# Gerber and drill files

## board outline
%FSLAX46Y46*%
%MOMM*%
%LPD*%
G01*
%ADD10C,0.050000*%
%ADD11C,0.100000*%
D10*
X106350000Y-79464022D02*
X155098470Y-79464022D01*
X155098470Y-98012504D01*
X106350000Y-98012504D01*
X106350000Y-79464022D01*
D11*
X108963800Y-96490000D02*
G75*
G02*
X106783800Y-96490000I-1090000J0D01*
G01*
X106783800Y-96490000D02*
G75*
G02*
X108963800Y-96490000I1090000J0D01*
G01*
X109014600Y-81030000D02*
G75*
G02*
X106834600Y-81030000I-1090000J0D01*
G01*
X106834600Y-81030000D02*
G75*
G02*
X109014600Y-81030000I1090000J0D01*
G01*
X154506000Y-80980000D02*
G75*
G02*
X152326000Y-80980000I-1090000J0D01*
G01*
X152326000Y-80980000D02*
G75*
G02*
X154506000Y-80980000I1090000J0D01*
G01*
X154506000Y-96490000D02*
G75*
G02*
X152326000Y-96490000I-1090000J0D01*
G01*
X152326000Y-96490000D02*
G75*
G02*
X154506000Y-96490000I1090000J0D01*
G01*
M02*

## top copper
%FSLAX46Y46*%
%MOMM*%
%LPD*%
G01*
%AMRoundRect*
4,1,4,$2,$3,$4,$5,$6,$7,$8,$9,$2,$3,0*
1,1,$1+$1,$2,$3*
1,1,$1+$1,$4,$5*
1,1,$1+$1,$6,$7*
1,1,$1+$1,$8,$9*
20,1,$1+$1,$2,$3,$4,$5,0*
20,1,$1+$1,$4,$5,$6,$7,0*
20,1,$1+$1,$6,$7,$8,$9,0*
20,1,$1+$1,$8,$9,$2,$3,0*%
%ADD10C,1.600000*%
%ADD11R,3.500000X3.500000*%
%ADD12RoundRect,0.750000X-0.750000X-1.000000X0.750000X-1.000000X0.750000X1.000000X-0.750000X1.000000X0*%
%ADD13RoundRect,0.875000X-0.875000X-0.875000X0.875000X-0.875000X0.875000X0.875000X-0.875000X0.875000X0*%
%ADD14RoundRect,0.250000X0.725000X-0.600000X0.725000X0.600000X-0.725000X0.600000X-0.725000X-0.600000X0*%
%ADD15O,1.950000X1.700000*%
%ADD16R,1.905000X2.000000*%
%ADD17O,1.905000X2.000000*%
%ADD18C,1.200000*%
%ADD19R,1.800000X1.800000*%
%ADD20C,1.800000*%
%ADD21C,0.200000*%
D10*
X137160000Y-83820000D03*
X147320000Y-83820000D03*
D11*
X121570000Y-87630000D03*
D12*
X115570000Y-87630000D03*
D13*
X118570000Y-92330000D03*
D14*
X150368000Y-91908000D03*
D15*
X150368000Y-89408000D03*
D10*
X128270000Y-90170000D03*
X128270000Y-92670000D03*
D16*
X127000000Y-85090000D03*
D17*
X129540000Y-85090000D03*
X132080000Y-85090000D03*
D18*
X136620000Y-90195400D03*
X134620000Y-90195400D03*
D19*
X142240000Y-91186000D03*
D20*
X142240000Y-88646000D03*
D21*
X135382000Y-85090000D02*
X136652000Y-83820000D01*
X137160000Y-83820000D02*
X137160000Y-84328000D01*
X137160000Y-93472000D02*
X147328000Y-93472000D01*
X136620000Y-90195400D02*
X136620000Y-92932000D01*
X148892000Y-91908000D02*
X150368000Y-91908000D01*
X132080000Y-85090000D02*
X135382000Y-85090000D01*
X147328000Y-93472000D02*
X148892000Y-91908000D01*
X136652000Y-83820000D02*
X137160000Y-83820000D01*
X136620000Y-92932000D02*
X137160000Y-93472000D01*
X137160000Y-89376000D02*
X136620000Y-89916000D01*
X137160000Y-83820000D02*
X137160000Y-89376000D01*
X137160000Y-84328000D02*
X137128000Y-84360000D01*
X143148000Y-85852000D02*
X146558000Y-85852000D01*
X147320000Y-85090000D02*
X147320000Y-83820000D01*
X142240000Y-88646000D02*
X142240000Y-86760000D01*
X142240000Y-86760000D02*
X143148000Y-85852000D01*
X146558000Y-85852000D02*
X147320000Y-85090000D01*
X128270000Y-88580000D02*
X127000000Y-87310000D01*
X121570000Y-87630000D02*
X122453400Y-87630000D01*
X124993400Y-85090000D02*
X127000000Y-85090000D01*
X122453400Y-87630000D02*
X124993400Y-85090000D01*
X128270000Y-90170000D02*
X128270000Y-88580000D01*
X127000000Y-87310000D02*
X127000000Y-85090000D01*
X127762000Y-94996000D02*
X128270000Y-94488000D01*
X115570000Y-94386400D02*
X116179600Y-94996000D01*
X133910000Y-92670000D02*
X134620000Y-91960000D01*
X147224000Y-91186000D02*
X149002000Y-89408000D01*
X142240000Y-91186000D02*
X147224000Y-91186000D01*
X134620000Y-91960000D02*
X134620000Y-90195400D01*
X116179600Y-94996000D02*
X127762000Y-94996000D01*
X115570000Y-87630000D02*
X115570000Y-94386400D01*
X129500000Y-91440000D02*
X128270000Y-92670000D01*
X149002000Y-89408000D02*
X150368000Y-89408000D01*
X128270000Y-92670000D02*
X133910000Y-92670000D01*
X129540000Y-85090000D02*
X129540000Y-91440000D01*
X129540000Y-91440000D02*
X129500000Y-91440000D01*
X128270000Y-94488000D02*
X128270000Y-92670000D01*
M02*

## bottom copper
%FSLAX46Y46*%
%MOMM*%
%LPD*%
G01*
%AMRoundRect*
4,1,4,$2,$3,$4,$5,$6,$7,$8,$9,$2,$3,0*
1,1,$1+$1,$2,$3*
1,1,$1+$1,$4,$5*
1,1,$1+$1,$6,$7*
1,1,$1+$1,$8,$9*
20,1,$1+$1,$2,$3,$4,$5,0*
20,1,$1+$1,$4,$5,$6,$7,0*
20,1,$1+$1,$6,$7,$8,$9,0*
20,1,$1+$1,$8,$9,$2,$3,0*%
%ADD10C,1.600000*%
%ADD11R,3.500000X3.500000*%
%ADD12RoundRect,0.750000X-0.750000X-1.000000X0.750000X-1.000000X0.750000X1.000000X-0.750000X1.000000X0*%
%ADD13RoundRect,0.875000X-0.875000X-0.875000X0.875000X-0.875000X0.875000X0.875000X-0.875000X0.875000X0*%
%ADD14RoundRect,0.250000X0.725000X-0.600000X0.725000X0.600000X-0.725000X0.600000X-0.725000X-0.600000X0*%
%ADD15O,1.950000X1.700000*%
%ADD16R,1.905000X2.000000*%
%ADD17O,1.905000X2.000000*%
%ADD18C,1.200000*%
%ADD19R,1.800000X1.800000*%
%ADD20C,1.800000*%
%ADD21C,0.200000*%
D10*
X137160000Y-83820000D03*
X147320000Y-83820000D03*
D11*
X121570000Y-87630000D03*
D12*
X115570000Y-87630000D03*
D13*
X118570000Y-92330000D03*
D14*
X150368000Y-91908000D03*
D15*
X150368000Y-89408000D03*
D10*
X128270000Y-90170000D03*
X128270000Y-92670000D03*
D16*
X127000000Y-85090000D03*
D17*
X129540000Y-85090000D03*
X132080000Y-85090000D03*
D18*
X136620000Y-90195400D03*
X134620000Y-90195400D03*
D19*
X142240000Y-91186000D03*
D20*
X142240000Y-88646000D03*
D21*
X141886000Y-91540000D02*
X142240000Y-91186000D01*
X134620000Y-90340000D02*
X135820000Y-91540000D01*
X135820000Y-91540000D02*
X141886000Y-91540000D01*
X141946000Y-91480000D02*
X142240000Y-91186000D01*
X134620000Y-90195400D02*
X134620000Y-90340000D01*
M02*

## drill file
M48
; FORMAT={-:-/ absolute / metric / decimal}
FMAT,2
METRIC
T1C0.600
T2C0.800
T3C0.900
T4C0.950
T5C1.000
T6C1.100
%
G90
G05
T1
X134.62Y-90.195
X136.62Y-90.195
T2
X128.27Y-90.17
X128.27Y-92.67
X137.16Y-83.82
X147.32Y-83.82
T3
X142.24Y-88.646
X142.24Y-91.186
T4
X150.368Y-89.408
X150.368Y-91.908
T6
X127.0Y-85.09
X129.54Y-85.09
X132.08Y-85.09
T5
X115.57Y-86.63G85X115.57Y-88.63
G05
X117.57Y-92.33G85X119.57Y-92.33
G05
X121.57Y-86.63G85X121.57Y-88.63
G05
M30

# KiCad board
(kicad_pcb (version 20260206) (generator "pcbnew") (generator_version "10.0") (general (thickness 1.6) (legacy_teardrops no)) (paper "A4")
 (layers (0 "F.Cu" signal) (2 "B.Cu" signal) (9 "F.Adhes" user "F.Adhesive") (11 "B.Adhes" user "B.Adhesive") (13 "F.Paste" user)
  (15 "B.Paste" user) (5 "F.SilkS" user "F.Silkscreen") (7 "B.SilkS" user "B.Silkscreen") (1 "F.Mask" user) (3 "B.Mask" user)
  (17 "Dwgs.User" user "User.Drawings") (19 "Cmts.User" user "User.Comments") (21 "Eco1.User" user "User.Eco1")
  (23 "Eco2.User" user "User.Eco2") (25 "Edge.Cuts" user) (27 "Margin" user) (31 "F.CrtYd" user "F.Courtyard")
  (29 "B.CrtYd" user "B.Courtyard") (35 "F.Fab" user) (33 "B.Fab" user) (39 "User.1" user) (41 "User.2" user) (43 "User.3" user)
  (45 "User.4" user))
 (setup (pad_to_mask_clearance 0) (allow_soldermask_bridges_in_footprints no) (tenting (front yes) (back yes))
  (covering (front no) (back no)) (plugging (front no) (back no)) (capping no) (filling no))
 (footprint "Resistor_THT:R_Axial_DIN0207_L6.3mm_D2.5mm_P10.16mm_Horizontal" (layer "F.Cu") (at 137.16 83.82)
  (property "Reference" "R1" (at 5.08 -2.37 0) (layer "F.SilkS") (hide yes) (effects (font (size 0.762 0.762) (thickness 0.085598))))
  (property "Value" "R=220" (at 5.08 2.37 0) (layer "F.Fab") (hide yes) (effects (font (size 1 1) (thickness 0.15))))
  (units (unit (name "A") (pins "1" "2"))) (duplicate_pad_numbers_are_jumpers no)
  (pad "1" thru_hole circle (at 0 0) (size 1.6 1.6) (drill 0.8) (layers "*.Cu" "*.Mask") (remove_unused_layers no) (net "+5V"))
  (pad "2" thru_hole circle (at 10.16 0) (size 1.6 1.6) (drill 0.8) (layers "*.Cu" "*.Mask") (remove_unused_layers no) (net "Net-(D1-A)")))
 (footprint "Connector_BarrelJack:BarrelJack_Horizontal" (layer "F.Cu") (at 121.57 87.63)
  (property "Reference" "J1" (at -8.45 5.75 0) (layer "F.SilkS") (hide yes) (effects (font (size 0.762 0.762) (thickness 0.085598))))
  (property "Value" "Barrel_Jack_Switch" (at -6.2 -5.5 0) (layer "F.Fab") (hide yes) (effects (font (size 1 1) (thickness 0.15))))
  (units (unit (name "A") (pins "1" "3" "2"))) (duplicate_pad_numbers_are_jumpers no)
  (pad "1" thru_hole rect (at 0 0) (size 3.5 3.5) (drill oval 1 3) (layers "*.Cu" "*.Mask") (remove_unused_layers no) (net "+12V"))
  (pad "2" thru_hole roundrect (at -6 0) (size 3 3.5) (drill oval 1 3) (layers "*.Cu" "*.Mask") (remove_unused_layers no)
   (roundrect_rratio 0.25) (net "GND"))
  (pad "3" thru_hole roundrect (at -3 4.7) (size 3.5 3.5) (drill oval 3 1) (layers "*.Cu" "*.Mask") (remove_unused_layers no)
   (roundrect_rratio 0.25) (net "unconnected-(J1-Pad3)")))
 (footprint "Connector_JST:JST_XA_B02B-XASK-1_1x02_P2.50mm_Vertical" (layer "F.Cu") (at 150.368 91.908 90)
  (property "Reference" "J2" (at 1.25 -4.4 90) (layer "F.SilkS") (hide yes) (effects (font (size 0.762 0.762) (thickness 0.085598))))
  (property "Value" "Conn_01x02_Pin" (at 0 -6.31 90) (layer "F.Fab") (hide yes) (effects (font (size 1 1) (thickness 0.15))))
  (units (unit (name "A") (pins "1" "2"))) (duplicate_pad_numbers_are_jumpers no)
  (pad "1" thru_hole roundrect (at 0 0 90) (size 1.7 1.95) (drill 0.95) (layers "*.Cu" "*.Mask") (remove_unused_layers no)
   (roundrect_rratio 0.147059) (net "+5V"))
  (pad "2" thru_hole oval (at 2.5 0 90) (size 1.7 1.95) (drill 0.95) (layers "*.Cu" "*.Mask") (remove_unused_layers no) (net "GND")))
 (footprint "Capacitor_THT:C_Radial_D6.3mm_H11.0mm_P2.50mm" (layer "F.Cu") (at 128.27 90.17 -90)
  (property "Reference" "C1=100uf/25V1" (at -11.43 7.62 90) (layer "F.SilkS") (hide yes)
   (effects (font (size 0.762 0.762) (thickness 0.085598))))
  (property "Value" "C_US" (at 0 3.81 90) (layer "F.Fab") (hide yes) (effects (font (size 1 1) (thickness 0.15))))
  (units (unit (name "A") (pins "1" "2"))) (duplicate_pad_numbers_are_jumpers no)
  (pad "1" thru_hole circle (at 0 0 270) (size 1.6 1.6) (drill 0.8) (layers "*.Cu" "*.Mask") (remove_unused_layers no) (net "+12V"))
  (pad "2" thru_hole circle (at 2.5 0 270) (size 1.6 1.6) (drill 0.8) (layers "*.Cu" "*.Mask") (remove_unused_layers no) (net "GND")))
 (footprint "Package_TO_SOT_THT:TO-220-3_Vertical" (layer "F.Cu") (at 127 85.09)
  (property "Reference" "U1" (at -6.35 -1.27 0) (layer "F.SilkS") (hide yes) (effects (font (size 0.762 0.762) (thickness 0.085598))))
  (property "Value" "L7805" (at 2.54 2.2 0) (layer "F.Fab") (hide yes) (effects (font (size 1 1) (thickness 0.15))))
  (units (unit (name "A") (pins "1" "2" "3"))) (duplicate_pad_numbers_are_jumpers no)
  (pad "1" thru_hole rect (at 0 0) (size 1.905 2) (drill 1.1) (layers "*.Cu" "*.Mask") (remove_unused_layers no) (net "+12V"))
  (pad "2" thru_hole oval (at 2.54 0) (size 1.905 2) (drill 1.1) (layers "*.Cu" "*.Mask") (remove_unused_layers no) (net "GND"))
  (pad "3" thru_hole oval (at 5.08 0) (size 1.905 2) (drill 1.1) (layers "*.Cu" "*.Mask") (remove_unused_layers no) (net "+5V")))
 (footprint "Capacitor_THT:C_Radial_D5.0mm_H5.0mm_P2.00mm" (layer "F.Cu") (at 136.62 90.1954 180)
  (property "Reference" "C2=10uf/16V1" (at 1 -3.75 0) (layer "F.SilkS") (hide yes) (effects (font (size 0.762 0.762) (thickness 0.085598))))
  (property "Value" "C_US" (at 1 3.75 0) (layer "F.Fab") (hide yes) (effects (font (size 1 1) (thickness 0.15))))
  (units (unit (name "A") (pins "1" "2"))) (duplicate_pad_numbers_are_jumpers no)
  (pad "1" thru_hole circle (at 0 0 180) (size 1.2 1.2) (drill 0.6) (layers "*.Cu" "*.Mask") (remove_unused_layers no) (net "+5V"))
  (pad "2" thru_hole circle (at 2 0 180) (size 1.2 1.2) (drill 0.6) (layers "*.Cu" "*.Mask") (remove_unused_layers no) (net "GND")))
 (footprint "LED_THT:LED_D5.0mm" (layer "F.Cu") (at 142.24 91.186 90)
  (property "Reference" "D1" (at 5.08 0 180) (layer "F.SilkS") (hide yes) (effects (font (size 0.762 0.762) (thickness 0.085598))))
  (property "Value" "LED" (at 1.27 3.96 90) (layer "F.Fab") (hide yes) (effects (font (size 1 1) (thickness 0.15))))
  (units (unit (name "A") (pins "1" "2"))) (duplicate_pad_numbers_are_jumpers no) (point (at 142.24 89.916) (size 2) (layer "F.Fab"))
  (pad "1" thru_hole rect (at 0 0 90) (size 1.8 1.8) (drill 0.9) (layers "*.Cu" "*.Mask") (remove_unused_layers no) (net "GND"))
  (pad "2" thru_hole circle (at 2.54 0 90) (size 1.8 1.8) (drill 0.9) (layers "*.Cu" "*.Mask") (remove_unused_layers no) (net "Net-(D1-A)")))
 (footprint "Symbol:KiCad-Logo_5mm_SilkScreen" (layer "B.Cu") (at 110.71 88.35 90)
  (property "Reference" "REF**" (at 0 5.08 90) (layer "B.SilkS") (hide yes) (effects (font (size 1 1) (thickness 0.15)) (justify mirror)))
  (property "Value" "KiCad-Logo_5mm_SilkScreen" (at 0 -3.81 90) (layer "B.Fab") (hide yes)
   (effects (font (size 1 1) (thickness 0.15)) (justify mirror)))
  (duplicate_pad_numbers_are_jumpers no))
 (gr_rect (start 106.35 79.464022) (end 155.09847 98.012504) (stroke (width 0.05) (type default)) (fill no) (layer "Edge.Cuts"))
 (gr_circle (center 107.8738 96.49) (end 108.9638 96.49) (stroke (width 0.1) (type solid)) (fill no) (layer "Edge.Cuts"))
 (gr_circle (center 107.9246 81.03) (end 109.0146 81.03) (stroke (width 0.1) (type solid)) (fill no) (layer "Edge.Cuts"))
 (gr_circle (center 153.416 80.98) (end 154.506 80.98) (stroke (width 0.1) (type solid)) (fill no) (layer "Edge.Cuts"))
 (gr_circle (center 153.416 96.49) (end 153.416 97.58) (stroke (width 0.1) (type solid)) (fill no) (layer "Edge.Cuts"))
 (segment (start 135.382 85.09) (end 136.652 83.82) (width 0.2) (layer "F.Cu") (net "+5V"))
 (segment (start 137.16 83.82) (end 137.16 84.328) (width 0.2) (layer "F.Cu") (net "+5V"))
 (segment (start 137.16 93.472) (end 147.328 93.472) (width 0.2) (layer "F.Cu") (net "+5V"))
 (segment (start 136.62 90.1954) (end 136.62 92.932) (width 0.2) (layer "F.Cu") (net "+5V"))
 (segment (start 148.892 91.908) (end 150.368 91.908) (width 0.2) (layer "F.Cu") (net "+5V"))
 (segment (start 132.08 85.09) (end 135.382 85.09) (width 0.2) (layer "F.Cu") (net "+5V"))
 (segment (start 147.328 93.472) (end 148.892 91.908) (width 0.2) (layer "F.Cu") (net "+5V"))
 (segment (start 136.652 83.82) (end 137.16 83.82) (width 0.2) (layer "F.Cu") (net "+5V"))
 (segment (start 136.62 92.932) (end 137.16 93.472) (width 0.2) (layer "F.Cu") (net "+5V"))
 (segment (start 137.16 89.376) (end 136.62 89.916) (width 0.2) (layer "F.Cu") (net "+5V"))
 (segment (start 137.16 83.82) (end 137.16 89.376) (width 0.2) (layer "F.Cu") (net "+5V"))
 (segment (start 137.16 84.328) (end 137.128 84.36) (width 0.2) (layer "F.Cu") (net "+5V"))
 (segment (start 143.148 85.852) (end 146.558 85.852) (width 0.2) (layer "F.Cu") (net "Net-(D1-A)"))
 (segment (start 147.32 85.09) (end 147.32 83.82) (width 0.2) (layer "F.Cu") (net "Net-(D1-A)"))
 (segment (start 142.24 88.646) (end 142.24 86.76) (width 0.2) (layer "F.Cu") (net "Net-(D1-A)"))
 (segment (start 142.24 86.76) (end 143.148 85.852) (width 0.2) (layer "F.Cu") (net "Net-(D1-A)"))
 (segment (start 146.558 85.852) (end 147.32 85.09) (width 0.2) (layer "F.Cu") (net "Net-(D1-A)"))
 (segment (start 128.27 88.58) (end 127 87.31) (width 0.2) (layer "F.Cu") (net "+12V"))
 (segment (start 121.57 87.63) (end 122.4534 87.63) (width 0.2) (layer "F.Cu") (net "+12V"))
 (segment (start 124.9934 85.09) (end 127 85.09) (width 0.2) (layer "F.Cu") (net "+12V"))
 (segment (start 122.4534 87.63) (end 124.9934 85.09) (width 0.2) (layer "F.Cu") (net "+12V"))
 (segment (start 128.27 90.17) (end 128.27 88.58) (width 0.2) (layer "F.Cu") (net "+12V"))
 (segment (start 127 87.31) (end 127 85.09) (width 0.2) (layer "F.Cu") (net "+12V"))
 (segment (start 127.762 94.996) (end 128.27 94.488) (width 0.2) (layer "F.Cu") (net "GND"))
 (segment (start 115.57 94.3864) (end 116.1796 94.996) (width 0.2) (layer "F.Cu") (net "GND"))
 (segment (start 133.91 92.67) (end 134.62 91.96) (width 0.2) (layer "F.Cu") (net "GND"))
 (segment (start 147.224 91.186) (end 149.002 89.408) (width 0.2) (layer "F.Cu") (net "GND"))
 (segment (start 142.24 91.186) (end 147.224 91.186) (width 0.2) (layer "F.Cu") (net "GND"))
 (segment (start 134.62 91.96) (end 134.62 90.1954) (width 0.2) (layer "F.Cu") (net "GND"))
 (segment (start 116.1796 94.996) (end 127.762 94.996) (width 0.2) (layer "F.Cu") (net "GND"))
 (segment (start 115.57 87.63) (end 115.57 94.3864) (width 0.2) (layer "F.Cu") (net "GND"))
 (segment (start 129.5 91.44) (end 128.27 92.67) (width 0.2) (layer "F.Cu") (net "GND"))
 (segment (start 149.002 89.408) (end 150.368 89.408) (width 0.2) (layer "F.Cu") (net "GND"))
 (segment (start 128.27 92.67) (end 133.91 92.67) (width 0.2) (layer "F.Cu") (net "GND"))
 (segment (start 129.54 85.09) (end 129.54 91.44) (width 0.2) (layer "F.Cu") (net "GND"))
 (segment (start 129.54 91.44) (end 129.5 91.44) (width 0.2) (layer "F.Cu") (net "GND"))
 (segment (start 128.27 94.488) (end 128.27 92.67) (width 0.2) (layer "F.Cu") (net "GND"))
 (segment (start 141.886 91.54) (end 142.24 91.186) (width 0.2) (layer "B.Cu") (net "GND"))
 (segment (start 134.62 90.34) (end 135.82 91.54) (width 0.2) (layer "B.Cu") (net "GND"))
 (segment (start 135.82 91.54) (end 141.886 91.54) (width 0.2) (layer "B.Cu") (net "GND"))
 (segment (start 141.946 91.48) (end 142.24 91.186) (width 0.2) (layer "B.Cu") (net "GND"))
 (segment (start 134.62 90.1954) (end 134.62 90.34) (width 0.2) (layer "B.Cu") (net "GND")))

